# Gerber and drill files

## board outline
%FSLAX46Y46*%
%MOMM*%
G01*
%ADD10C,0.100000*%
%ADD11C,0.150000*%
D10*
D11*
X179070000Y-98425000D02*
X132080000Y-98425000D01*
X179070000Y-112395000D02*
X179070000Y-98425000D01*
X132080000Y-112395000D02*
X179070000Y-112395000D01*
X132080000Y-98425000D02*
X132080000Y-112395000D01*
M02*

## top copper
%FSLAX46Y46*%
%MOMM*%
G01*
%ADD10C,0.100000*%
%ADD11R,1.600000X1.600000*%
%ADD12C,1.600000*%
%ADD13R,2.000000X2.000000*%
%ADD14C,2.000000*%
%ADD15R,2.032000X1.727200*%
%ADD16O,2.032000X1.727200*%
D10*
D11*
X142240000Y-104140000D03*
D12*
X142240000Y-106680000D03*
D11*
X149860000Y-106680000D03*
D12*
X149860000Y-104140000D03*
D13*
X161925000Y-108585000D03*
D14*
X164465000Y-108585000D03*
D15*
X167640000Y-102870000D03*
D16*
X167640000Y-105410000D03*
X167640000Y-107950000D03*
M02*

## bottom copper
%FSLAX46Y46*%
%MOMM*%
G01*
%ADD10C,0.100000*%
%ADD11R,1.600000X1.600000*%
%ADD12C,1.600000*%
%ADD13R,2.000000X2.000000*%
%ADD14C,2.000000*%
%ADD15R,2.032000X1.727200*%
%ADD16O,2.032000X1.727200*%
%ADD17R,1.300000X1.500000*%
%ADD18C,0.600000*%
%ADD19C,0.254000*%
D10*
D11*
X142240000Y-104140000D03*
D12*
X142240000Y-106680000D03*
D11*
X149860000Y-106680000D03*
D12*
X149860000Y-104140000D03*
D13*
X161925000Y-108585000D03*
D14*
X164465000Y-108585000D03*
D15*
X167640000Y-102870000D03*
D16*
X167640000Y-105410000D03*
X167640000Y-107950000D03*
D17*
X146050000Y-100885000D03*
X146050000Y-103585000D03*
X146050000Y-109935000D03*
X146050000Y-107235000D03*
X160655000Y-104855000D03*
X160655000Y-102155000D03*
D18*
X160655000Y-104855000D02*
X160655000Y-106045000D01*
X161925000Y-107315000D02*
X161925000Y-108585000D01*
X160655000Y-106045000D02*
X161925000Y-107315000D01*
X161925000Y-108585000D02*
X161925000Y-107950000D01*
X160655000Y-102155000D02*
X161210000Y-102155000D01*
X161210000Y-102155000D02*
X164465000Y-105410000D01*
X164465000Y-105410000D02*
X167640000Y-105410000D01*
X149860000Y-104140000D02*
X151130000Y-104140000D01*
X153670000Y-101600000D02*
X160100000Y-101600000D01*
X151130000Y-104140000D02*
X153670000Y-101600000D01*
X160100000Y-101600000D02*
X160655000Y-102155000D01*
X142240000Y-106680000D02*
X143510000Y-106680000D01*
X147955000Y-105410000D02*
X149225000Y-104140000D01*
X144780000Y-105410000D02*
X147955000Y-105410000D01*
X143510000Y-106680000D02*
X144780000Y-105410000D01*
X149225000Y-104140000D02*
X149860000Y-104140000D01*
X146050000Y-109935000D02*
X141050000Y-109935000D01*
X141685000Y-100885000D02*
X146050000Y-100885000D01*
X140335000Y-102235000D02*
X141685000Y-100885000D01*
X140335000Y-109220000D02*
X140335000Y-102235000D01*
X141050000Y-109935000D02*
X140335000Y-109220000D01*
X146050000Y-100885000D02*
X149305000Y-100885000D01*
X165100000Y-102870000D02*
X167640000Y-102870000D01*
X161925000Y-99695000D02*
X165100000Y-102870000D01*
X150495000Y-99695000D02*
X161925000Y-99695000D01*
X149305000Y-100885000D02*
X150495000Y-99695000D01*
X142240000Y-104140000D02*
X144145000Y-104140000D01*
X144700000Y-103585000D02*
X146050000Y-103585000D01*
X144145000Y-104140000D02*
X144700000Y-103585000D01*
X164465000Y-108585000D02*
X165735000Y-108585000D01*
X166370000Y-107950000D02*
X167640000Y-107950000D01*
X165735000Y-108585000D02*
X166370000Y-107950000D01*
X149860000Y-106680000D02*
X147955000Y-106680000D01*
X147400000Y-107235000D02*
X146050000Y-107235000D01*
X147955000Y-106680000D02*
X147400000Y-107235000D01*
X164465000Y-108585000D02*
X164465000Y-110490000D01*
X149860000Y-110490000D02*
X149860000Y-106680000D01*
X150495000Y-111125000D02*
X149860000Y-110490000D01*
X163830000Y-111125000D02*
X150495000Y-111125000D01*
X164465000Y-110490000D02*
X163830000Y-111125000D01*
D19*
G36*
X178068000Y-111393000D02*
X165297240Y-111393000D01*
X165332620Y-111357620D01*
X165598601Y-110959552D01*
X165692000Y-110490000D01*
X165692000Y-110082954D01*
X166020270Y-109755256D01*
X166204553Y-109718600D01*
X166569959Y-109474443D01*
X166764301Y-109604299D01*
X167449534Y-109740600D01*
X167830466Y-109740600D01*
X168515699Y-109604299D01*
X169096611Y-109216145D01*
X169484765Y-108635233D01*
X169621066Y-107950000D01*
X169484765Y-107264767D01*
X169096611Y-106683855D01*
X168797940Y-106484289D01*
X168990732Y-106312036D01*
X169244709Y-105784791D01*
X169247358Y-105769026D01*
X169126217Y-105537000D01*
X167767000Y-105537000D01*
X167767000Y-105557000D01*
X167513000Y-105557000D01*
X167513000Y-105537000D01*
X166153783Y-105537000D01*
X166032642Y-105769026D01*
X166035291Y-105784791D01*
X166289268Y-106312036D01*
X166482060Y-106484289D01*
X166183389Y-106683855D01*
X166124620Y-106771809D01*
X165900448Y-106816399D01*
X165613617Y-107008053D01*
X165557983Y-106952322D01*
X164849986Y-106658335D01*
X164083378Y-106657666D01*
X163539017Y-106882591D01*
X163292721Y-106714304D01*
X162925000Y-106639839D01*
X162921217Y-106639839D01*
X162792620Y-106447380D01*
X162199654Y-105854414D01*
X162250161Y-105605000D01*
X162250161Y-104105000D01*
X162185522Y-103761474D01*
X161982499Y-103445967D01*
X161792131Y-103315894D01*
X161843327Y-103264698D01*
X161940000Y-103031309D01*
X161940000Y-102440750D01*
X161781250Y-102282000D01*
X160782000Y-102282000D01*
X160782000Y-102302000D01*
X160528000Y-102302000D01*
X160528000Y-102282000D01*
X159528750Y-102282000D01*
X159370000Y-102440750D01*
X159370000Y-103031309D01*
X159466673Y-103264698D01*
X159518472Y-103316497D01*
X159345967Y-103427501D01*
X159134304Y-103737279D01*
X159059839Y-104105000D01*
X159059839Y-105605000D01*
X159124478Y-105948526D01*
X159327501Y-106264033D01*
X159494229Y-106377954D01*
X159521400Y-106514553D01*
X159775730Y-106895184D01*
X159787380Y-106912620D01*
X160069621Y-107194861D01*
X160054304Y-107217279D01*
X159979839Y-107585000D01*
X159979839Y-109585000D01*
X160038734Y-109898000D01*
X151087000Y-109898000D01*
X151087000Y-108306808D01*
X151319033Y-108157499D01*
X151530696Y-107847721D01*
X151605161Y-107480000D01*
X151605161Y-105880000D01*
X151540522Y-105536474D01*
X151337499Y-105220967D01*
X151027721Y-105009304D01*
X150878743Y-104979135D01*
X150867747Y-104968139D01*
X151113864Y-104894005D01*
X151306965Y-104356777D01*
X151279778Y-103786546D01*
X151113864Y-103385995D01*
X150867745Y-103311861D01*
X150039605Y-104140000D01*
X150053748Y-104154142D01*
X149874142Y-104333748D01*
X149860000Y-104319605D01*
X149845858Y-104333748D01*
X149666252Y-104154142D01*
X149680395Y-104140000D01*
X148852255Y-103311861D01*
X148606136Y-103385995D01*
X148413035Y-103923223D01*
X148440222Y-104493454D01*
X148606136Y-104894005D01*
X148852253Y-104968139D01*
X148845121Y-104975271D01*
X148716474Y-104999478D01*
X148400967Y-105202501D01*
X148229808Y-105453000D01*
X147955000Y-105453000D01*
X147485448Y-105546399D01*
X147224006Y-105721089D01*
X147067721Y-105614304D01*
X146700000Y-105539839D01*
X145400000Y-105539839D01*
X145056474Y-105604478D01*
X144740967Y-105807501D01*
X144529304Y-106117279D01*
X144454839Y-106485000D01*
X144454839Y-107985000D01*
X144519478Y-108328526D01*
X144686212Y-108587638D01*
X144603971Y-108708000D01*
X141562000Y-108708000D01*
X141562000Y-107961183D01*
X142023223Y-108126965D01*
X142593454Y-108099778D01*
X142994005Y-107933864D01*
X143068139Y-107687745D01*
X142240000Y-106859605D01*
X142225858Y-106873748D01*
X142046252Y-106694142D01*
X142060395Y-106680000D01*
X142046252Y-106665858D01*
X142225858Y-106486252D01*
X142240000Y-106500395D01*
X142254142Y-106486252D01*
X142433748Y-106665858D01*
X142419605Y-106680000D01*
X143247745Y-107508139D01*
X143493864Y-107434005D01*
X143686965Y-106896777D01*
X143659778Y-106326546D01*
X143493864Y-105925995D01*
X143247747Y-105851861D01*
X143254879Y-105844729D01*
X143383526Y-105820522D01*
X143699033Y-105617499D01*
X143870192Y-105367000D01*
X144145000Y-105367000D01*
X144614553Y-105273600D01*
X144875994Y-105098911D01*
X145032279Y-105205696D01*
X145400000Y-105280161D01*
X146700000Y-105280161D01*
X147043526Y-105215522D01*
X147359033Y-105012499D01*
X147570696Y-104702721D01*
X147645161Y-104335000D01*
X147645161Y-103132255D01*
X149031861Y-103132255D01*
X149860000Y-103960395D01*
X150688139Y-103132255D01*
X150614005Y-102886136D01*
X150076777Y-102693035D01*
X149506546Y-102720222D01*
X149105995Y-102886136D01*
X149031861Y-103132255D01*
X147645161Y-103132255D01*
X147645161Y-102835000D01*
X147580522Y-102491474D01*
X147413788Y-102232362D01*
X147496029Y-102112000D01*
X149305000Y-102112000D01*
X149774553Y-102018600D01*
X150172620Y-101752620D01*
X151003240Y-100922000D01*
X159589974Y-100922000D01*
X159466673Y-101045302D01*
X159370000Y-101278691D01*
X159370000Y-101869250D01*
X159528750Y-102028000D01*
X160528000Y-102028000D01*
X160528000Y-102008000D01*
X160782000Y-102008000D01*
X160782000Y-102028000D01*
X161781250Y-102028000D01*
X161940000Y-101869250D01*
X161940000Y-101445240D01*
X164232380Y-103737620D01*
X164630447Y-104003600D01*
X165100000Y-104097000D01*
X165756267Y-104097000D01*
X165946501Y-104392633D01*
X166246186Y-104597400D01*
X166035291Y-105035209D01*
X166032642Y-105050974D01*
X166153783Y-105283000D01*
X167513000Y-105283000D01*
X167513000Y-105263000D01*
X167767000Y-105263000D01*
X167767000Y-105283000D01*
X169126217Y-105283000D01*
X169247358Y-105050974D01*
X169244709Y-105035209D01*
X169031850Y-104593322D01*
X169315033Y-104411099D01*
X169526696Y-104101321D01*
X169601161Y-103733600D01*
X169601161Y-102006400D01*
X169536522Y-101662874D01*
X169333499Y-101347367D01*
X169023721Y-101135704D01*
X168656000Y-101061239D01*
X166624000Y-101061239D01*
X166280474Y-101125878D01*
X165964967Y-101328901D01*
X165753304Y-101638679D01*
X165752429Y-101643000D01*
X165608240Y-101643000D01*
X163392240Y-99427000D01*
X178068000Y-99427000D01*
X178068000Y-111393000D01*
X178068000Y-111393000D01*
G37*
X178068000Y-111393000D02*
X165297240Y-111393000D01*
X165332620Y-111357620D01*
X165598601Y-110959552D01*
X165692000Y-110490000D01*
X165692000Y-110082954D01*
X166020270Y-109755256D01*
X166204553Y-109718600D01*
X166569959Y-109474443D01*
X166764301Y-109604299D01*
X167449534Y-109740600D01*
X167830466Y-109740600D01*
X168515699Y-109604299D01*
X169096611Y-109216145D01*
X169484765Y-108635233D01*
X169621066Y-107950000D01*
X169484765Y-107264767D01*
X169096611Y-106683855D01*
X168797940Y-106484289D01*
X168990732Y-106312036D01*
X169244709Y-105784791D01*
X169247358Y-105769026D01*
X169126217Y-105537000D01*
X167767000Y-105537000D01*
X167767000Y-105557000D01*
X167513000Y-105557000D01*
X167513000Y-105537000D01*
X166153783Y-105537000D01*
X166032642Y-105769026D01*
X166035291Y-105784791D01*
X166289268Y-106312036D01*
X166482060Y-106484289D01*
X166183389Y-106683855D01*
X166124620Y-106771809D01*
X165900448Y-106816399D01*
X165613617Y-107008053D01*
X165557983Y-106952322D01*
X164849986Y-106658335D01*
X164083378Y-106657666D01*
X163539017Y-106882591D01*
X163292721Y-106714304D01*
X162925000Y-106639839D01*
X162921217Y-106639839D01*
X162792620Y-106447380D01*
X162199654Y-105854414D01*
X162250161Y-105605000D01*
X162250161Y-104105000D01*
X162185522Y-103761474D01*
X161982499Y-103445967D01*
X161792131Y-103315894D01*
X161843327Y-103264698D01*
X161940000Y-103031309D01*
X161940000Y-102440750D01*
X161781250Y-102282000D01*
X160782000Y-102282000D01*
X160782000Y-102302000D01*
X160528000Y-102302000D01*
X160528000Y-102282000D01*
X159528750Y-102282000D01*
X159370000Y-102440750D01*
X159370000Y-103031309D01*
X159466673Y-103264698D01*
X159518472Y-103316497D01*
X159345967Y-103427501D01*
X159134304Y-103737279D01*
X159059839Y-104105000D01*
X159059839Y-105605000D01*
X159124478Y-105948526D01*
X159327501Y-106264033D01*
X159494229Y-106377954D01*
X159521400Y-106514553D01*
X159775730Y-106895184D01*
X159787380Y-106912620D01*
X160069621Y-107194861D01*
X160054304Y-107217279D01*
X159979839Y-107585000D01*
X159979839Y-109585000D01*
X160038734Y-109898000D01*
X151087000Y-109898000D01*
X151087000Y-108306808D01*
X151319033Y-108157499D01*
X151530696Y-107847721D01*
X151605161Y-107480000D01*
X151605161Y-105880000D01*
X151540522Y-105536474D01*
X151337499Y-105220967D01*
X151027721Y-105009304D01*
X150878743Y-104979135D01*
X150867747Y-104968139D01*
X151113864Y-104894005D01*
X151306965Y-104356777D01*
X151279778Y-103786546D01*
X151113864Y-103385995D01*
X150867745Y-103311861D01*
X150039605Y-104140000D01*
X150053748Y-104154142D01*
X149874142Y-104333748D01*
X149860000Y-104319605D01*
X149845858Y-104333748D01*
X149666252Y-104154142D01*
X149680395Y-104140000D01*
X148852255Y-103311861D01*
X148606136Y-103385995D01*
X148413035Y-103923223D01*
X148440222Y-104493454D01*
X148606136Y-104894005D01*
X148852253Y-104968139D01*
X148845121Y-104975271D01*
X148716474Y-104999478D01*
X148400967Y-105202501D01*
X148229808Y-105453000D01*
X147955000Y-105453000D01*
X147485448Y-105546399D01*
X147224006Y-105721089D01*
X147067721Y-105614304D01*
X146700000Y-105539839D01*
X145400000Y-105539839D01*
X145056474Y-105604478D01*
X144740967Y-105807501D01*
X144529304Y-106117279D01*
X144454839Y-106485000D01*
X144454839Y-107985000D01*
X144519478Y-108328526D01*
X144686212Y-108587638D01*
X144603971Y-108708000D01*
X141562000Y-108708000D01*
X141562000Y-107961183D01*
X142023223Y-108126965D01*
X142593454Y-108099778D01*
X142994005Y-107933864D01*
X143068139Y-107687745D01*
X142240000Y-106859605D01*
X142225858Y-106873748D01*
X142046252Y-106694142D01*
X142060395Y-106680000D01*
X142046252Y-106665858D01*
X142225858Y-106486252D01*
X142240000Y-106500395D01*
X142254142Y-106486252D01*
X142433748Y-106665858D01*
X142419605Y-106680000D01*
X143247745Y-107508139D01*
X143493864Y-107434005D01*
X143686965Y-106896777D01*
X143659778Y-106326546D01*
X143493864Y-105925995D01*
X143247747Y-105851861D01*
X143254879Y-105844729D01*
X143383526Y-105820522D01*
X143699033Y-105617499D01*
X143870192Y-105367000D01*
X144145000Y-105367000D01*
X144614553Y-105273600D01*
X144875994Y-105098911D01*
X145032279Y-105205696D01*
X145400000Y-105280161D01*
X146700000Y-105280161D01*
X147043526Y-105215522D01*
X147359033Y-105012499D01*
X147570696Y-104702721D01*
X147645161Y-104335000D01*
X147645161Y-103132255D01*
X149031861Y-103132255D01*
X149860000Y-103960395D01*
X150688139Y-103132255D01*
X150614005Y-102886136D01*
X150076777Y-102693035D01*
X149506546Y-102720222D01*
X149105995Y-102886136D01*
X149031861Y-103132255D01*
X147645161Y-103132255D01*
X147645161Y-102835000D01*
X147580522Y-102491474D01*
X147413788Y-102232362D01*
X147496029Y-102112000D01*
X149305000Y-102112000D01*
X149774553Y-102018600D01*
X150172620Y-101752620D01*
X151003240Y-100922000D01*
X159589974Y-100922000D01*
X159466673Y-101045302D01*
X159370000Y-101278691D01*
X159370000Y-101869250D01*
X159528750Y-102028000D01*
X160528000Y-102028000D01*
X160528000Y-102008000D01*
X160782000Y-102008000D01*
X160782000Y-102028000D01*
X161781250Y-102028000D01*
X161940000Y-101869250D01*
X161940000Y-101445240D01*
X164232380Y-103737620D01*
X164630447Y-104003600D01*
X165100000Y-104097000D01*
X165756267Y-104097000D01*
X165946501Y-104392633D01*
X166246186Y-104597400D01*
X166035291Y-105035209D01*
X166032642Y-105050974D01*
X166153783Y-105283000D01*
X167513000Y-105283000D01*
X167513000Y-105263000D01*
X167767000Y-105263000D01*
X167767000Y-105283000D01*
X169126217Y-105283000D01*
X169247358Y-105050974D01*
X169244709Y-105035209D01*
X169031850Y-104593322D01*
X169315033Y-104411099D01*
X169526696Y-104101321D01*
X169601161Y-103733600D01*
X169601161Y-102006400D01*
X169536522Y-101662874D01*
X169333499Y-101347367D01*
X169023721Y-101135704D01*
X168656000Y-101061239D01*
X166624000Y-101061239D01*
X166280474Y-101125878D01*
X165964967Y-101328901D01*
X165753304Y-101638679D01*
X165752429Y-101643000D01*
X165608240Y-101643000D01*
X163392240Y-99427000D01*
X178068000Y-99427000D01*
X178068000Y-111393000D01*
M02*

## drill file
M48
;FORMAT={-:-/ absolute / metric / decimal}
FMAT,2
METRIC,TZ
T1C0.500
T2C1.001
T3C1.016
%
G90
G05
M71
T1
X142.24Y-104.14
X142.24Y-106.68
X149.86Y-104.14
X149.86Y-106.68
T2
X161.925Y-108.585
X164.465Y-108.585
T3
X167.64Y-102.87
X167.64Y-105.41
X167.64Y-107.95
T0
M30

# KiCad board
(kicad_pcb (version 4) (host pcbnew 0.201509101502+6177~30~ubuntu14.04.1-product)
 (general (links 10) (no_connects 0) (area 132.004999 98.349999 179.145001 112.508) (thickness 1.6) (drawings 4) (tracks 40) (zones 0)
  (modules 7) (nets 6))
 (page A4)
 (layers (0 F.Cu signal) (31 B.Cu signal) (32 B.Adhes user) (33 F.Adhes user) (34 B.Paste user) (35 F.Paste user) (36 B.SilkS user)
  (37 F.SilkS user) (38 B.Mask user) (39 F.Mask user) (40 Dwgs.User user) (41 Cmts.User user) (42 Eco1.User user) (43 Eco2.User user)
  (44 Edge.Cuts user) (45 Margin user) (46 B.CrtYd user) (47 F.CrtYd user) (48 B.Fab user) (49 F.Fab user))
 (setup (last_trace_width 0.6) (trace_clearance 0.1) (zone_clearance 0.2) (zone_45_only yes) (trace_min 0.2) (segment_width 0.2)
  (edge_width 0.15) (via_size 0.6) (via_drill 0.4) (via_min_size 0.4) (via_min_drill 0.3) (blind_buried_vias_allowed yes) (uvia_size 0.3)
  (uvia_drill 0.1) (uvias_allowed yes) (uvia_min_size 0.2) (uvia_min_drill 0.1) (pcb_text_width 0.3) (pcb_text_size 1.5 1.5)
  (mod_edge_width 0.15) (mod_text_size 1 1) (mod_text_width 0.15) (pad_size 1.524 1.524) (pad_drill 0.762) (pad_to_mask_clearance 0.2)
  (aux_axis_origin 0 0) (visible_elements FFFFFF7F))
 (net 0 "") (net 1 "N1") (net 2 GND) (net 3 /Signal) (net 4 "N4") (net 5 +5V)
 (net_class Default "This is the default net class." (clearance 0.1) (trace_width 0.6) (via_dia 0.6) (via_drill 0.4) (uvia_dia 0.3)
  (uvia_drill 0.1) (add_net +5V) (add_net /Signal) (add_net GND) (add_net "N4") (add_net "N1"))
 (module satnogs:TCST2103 (layer F.Cu) (at 146.05 105.41)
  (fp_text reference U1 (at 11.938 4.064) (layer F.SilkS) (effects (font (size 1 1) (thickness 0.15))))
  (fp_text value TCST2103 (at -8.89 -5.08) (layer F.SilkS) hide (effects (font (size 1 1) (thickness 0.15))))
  (pad 1 thru_hole rect (at -3.81 -1.27) (size 1.6 1.6) (drill 0.5) (layers *.Cu *.Mask F.SilkS) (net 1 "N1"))
  (pad 2 thru_hole circle (at -3.81 1.27) (size 1.6 1.6) (drill 0.5) (layers *.Cu *.Mask F.SilkS) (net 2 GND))
  (pad 3 thru_hole rect (at 3.81 1.27) (size 1.6 1.6) (drill 0.5) (layers *.Cu *.Mask F.SilkS) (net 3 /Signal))
  (pad 4 thru_hole circle (at 3.81 -1.27) (size 1.6 1.6) (drill 0.5) (layers *.Cu *.Mask F.SilkS) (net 2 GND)))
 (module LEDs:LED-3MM (layer F.Cu) (at 161.925 108.585)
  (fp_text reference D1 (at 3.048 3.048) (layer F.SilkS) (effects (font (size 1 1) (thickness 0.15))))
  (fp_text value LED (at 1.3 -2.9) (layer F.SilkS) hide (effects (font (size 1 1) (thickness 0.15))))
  (pad 1 thru_hole rect (at 0 0 90) (size 2 2) (drill 1.00076) (layers *.Cu *.Mask F.SilkS) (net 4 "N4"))
  (pad 2 thru_hole circle (at 2.54 0) (size 2 2) (drill 1.00076) (layers *.Cu *.Mask F.SilkS) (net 3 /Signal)))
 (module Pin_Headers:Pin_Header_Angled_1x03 (layer F.Cu) (at 167.64 102.87)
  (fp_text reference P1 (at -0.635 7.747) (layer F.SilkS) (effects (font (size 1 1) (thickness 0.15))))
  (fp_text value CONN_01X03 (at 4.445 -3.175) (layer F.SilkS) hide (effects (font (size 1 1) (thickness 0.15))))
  (pad 1 thru_hole rect (at 0 0) (size 2.032 1.7272) (drill 1.016) (layers *.Cu *.Mask F.SilkS) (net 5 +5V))
  (pad 2 thru_hole oval (at 0 2.54) (size 2.032 1.7272) (drill 1.016) (layers *.Cu *.Mask F.SilkS) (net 2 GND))
  (pad 3 thru_hole oval (at 0 5.08) (size 2.032 1.7272) (drill 1.016) (layers *.Cu *.Mask F.SilkS) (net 3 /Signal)))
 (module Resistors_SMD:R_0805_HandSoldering (layer B.Cu) (at 146.05 102.235 270)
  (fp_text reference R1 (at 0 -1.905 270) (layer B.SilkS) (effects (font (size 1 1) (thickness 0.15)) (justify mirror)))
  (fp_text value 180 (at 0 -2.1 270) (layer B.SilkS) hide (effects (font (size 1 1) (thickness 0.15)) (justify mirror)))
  (pad 1 smd rect (at -1.35 0 270) (size 1.5 1.3) (layers B.Cu B.Paste B.Mask) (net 5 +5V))
  (pad 2 smd rect (at 1.35 0 270) (size 1.5 1.3) (layers B.Cu B.Paste B.Mask) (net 1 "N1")))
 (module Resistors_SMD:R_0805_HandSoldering (layer B.Cu) (at 146.05 108.585 90)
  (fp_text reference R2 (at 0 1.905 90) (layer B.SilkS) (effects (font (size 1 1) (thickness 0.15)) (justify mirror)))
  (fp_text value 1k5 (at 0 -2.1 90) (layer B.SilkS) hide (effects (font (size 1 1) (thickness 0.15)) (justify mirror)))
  (pad 1 smd rect (at -1.35 0 90) (size 1.5 1.3) (layers B.Cu B.Paste B.Mask) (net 5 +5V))
  (pad 2 smd rect (at 1.35 0 90) (size 1.5 1.3) (layers B.Cu B.Paste B.Mask) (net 3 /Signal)))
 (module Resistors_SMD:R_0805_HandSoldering (layer B.Cu) (at 160.655 103.505 90)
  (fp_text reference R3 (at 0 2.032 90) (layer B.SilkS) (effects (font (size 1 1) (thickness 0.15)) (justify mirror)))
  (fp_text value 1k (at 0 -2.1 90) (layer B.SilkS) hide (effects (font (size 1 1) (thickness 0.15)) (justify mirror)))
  (pad 1 smd rect (at -1.35 0 90) (size 1.5 1.3) (layers B.Cu B.Paste B.Mask) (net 4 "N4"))
  (pad 2 smd rect (at 1.35 0 90) (size 1.5 1.3) (layers B.Cu B.Paste B.Mask) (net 2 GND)))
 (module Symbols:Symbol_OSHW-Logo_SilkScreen (layer B.Cu) (at 136.525 105.41 180)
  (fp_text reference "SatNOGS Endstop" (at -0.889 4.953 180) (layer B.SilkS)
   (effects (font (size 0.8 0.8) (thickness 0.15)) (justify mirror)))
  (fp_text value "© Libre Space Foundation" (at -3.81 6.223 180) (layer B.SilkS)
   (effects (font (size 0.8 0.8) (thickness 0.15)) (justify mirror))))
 (gr_line (start 179.07 98.425) (end 132.08 98.425) (angle 90) (layer Edge.Cuts) (width 0.15))
 (gr_line (start 179.07 112.395) (end 179.07 98.425) (angle 90) (layer Edge.Cuts) (width 0.15))
 (gr_line (start 132.08 112.395) (end 179.07 112.395) (angle 90) (layer Edge.Cuts) (width 0.15))
 (gr_line (start 132.08 98.425) (end 132.08 112.395) (angle 90) (layer Edge.Cuts) (width 0.15))
 (segment (start 160.655 104.855) (end 160.655 106.045) (width 0.6) (layer B.Cu) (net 4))
 (segment (start 161.925 107.315) (end 161.925 108.585) (width 0.6) (layer B.Cu) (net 4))
 (segment (start 160.655 106.045) (end 161.925 107.315) (width 0.6) (layer B.Cu) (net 4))
 (segment (start 161.925 108.585) (end 161.925 107.95) (width 0.6) (layer B.Cu) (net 4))
 (segment (start 160.655 102.155) (end 161.21 102.155) (width 0.6) (layer B.Cu) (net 2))
 (segment (start 161.21 102.155) (end 164.465 105.41) (width 0.6) (layer B.Cu) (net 2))
 (segment (start 164.465 105.41) (end 167.64 105.41) (width 0.6) (layer B.Cu) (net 2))
 (segment (start 149.86 104.14) (end 151.13 104.14) (width 0.6) (layer B.Cu) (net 2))
 (segment (start 153.67 101.6) (end 160.1 101.6) (width 0.6) (layer B.Cu) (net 2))
 (segment (start 151.13 104.14) (end 153.67 101.6) (width 0.6) (layer B.Cu) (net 2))
 (segment (start 160.1 101.6) (end 160.655 102.155) (width 0.6) (layer B.Cu) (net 2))
 (segment (start 142.24 106.68) (end 143.51 106.68) (width 0.6) (layer B.Cu) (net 2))
 (segment (start 147.955 105.41) (end 149.225 104.14) (width 0.6) (layer B.Cu) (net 2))
 (segment (start 144.78 105.41) (end 147.955 105.41) (width 0.6) (layer B.Cu) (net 2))
 (segment (start 143.51 106.68) (end 144.78 105.41) (width 0.6) (layer B.Cu) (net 2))
 (segment (start 149.225 104.14) (end 149.86 104.14) (width 0.6) (layer B.Cu) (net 2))
 (segment (start 146.05 109.935) (end 141.05 109.935) (width 0.6) (layer B.Cu) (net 5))
 (segment (start 141.685 100.885) (end 146.05 100.885) (width 0.6) (layer B.Cu) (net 5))
 (segment (start 140.335 102.235) (end 141.685 100.885) (width 0.6) (layer B.Cu) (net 5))
 (segment (start 140.335 109.22) (end 140.335 102.235) (width 0.6) (layer B.Cu) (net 5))
 (segment (start 141.05 109.935) (end 140.335 109.22) (width 0.6) (layer B.Cu) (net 5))
 (segment (start 146.05 100.885) (end 149.305 100.885) (width 0.6) (layer B.Cu) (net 5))
 (segment (start 165.1 102.87) (end 167.64 102.87) (width 0.6) (layer B.Cu) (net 5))
 (segment (start 161.925 99.695) (end 165.1 102.87) (width 0.6) (layer B.Cu) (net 5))
 (segment (start 150.495 99.695) (end 161.925 99.695) (width 0.6) (layer B.Cu) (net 5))
 (segment (start 149.305 100.885) (end 150.495 99.695) (width 0.6) (layer B.Cu) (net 5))
 (segment (start 142.24 104.14) (end 144.145 104.14) (width 0.6) (layer B.Cu) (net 1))
 (segment (start 144.7 103.585) (end 146.05 103.585) (width 0.6) (layer B.Cu) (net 1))
 (segment (start 144.145 104.14) (end 144.7 103.585) (width 0.6) (layer B.Cu) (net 1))
 (segment (start 164.465 108.585) (end 165.735 108.585) (width 0.6) (layer B.Cu) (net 3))
 (segment (start 166.37 107.95) (end 167.64 107.95) (width 0.6) (layer B.Cu) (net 3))
 (segment (start 165.735 108.585) (end 166.37 107.95) (width 0.6) (layer B.Cu) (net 3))
 (segment (start 149.86 106.68) (end 147.955 106.68) (width 0.6) (layer B.Cu) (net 3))
 (segment (start 147.4 107.235) (end 146.05 107.235) (width 0.6) (layer B.Cu) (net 3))
 (segment (start 147.955 106.68) (end 147.4 107.235) (width 0.6) (layer B.Cu) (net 3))
 (segment (start 164.465 108.585) (end 164.465 110.49) (width 0.6) (layer B.Cu) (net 3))
 (segment (start 149.86 110.49) (end 149.86 106.68) (width 0.6) (layer B.Cu) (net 3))
 (segment (start 150.495 111.125) (end 149.86 110.49) (width 0.6) (layer B.Cu) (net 3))
 (segment (start 163.83 111.125) (end 150.495 111.125) (width 0.6) (layer B.Cu) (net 3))
 (segment (start 164.465 110.49) (end 163.83 111.125) (width 0.6) (layer B.Cu) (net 3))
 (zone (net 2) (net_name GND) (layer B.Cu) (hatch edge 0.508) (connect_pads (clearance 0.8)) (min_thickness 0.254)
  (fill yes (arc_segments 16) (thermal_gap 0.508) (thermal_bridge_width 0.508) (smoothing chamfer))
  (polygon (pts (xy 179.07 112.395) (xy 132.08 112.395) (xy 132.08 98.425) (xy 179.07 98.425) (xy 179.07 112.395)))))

